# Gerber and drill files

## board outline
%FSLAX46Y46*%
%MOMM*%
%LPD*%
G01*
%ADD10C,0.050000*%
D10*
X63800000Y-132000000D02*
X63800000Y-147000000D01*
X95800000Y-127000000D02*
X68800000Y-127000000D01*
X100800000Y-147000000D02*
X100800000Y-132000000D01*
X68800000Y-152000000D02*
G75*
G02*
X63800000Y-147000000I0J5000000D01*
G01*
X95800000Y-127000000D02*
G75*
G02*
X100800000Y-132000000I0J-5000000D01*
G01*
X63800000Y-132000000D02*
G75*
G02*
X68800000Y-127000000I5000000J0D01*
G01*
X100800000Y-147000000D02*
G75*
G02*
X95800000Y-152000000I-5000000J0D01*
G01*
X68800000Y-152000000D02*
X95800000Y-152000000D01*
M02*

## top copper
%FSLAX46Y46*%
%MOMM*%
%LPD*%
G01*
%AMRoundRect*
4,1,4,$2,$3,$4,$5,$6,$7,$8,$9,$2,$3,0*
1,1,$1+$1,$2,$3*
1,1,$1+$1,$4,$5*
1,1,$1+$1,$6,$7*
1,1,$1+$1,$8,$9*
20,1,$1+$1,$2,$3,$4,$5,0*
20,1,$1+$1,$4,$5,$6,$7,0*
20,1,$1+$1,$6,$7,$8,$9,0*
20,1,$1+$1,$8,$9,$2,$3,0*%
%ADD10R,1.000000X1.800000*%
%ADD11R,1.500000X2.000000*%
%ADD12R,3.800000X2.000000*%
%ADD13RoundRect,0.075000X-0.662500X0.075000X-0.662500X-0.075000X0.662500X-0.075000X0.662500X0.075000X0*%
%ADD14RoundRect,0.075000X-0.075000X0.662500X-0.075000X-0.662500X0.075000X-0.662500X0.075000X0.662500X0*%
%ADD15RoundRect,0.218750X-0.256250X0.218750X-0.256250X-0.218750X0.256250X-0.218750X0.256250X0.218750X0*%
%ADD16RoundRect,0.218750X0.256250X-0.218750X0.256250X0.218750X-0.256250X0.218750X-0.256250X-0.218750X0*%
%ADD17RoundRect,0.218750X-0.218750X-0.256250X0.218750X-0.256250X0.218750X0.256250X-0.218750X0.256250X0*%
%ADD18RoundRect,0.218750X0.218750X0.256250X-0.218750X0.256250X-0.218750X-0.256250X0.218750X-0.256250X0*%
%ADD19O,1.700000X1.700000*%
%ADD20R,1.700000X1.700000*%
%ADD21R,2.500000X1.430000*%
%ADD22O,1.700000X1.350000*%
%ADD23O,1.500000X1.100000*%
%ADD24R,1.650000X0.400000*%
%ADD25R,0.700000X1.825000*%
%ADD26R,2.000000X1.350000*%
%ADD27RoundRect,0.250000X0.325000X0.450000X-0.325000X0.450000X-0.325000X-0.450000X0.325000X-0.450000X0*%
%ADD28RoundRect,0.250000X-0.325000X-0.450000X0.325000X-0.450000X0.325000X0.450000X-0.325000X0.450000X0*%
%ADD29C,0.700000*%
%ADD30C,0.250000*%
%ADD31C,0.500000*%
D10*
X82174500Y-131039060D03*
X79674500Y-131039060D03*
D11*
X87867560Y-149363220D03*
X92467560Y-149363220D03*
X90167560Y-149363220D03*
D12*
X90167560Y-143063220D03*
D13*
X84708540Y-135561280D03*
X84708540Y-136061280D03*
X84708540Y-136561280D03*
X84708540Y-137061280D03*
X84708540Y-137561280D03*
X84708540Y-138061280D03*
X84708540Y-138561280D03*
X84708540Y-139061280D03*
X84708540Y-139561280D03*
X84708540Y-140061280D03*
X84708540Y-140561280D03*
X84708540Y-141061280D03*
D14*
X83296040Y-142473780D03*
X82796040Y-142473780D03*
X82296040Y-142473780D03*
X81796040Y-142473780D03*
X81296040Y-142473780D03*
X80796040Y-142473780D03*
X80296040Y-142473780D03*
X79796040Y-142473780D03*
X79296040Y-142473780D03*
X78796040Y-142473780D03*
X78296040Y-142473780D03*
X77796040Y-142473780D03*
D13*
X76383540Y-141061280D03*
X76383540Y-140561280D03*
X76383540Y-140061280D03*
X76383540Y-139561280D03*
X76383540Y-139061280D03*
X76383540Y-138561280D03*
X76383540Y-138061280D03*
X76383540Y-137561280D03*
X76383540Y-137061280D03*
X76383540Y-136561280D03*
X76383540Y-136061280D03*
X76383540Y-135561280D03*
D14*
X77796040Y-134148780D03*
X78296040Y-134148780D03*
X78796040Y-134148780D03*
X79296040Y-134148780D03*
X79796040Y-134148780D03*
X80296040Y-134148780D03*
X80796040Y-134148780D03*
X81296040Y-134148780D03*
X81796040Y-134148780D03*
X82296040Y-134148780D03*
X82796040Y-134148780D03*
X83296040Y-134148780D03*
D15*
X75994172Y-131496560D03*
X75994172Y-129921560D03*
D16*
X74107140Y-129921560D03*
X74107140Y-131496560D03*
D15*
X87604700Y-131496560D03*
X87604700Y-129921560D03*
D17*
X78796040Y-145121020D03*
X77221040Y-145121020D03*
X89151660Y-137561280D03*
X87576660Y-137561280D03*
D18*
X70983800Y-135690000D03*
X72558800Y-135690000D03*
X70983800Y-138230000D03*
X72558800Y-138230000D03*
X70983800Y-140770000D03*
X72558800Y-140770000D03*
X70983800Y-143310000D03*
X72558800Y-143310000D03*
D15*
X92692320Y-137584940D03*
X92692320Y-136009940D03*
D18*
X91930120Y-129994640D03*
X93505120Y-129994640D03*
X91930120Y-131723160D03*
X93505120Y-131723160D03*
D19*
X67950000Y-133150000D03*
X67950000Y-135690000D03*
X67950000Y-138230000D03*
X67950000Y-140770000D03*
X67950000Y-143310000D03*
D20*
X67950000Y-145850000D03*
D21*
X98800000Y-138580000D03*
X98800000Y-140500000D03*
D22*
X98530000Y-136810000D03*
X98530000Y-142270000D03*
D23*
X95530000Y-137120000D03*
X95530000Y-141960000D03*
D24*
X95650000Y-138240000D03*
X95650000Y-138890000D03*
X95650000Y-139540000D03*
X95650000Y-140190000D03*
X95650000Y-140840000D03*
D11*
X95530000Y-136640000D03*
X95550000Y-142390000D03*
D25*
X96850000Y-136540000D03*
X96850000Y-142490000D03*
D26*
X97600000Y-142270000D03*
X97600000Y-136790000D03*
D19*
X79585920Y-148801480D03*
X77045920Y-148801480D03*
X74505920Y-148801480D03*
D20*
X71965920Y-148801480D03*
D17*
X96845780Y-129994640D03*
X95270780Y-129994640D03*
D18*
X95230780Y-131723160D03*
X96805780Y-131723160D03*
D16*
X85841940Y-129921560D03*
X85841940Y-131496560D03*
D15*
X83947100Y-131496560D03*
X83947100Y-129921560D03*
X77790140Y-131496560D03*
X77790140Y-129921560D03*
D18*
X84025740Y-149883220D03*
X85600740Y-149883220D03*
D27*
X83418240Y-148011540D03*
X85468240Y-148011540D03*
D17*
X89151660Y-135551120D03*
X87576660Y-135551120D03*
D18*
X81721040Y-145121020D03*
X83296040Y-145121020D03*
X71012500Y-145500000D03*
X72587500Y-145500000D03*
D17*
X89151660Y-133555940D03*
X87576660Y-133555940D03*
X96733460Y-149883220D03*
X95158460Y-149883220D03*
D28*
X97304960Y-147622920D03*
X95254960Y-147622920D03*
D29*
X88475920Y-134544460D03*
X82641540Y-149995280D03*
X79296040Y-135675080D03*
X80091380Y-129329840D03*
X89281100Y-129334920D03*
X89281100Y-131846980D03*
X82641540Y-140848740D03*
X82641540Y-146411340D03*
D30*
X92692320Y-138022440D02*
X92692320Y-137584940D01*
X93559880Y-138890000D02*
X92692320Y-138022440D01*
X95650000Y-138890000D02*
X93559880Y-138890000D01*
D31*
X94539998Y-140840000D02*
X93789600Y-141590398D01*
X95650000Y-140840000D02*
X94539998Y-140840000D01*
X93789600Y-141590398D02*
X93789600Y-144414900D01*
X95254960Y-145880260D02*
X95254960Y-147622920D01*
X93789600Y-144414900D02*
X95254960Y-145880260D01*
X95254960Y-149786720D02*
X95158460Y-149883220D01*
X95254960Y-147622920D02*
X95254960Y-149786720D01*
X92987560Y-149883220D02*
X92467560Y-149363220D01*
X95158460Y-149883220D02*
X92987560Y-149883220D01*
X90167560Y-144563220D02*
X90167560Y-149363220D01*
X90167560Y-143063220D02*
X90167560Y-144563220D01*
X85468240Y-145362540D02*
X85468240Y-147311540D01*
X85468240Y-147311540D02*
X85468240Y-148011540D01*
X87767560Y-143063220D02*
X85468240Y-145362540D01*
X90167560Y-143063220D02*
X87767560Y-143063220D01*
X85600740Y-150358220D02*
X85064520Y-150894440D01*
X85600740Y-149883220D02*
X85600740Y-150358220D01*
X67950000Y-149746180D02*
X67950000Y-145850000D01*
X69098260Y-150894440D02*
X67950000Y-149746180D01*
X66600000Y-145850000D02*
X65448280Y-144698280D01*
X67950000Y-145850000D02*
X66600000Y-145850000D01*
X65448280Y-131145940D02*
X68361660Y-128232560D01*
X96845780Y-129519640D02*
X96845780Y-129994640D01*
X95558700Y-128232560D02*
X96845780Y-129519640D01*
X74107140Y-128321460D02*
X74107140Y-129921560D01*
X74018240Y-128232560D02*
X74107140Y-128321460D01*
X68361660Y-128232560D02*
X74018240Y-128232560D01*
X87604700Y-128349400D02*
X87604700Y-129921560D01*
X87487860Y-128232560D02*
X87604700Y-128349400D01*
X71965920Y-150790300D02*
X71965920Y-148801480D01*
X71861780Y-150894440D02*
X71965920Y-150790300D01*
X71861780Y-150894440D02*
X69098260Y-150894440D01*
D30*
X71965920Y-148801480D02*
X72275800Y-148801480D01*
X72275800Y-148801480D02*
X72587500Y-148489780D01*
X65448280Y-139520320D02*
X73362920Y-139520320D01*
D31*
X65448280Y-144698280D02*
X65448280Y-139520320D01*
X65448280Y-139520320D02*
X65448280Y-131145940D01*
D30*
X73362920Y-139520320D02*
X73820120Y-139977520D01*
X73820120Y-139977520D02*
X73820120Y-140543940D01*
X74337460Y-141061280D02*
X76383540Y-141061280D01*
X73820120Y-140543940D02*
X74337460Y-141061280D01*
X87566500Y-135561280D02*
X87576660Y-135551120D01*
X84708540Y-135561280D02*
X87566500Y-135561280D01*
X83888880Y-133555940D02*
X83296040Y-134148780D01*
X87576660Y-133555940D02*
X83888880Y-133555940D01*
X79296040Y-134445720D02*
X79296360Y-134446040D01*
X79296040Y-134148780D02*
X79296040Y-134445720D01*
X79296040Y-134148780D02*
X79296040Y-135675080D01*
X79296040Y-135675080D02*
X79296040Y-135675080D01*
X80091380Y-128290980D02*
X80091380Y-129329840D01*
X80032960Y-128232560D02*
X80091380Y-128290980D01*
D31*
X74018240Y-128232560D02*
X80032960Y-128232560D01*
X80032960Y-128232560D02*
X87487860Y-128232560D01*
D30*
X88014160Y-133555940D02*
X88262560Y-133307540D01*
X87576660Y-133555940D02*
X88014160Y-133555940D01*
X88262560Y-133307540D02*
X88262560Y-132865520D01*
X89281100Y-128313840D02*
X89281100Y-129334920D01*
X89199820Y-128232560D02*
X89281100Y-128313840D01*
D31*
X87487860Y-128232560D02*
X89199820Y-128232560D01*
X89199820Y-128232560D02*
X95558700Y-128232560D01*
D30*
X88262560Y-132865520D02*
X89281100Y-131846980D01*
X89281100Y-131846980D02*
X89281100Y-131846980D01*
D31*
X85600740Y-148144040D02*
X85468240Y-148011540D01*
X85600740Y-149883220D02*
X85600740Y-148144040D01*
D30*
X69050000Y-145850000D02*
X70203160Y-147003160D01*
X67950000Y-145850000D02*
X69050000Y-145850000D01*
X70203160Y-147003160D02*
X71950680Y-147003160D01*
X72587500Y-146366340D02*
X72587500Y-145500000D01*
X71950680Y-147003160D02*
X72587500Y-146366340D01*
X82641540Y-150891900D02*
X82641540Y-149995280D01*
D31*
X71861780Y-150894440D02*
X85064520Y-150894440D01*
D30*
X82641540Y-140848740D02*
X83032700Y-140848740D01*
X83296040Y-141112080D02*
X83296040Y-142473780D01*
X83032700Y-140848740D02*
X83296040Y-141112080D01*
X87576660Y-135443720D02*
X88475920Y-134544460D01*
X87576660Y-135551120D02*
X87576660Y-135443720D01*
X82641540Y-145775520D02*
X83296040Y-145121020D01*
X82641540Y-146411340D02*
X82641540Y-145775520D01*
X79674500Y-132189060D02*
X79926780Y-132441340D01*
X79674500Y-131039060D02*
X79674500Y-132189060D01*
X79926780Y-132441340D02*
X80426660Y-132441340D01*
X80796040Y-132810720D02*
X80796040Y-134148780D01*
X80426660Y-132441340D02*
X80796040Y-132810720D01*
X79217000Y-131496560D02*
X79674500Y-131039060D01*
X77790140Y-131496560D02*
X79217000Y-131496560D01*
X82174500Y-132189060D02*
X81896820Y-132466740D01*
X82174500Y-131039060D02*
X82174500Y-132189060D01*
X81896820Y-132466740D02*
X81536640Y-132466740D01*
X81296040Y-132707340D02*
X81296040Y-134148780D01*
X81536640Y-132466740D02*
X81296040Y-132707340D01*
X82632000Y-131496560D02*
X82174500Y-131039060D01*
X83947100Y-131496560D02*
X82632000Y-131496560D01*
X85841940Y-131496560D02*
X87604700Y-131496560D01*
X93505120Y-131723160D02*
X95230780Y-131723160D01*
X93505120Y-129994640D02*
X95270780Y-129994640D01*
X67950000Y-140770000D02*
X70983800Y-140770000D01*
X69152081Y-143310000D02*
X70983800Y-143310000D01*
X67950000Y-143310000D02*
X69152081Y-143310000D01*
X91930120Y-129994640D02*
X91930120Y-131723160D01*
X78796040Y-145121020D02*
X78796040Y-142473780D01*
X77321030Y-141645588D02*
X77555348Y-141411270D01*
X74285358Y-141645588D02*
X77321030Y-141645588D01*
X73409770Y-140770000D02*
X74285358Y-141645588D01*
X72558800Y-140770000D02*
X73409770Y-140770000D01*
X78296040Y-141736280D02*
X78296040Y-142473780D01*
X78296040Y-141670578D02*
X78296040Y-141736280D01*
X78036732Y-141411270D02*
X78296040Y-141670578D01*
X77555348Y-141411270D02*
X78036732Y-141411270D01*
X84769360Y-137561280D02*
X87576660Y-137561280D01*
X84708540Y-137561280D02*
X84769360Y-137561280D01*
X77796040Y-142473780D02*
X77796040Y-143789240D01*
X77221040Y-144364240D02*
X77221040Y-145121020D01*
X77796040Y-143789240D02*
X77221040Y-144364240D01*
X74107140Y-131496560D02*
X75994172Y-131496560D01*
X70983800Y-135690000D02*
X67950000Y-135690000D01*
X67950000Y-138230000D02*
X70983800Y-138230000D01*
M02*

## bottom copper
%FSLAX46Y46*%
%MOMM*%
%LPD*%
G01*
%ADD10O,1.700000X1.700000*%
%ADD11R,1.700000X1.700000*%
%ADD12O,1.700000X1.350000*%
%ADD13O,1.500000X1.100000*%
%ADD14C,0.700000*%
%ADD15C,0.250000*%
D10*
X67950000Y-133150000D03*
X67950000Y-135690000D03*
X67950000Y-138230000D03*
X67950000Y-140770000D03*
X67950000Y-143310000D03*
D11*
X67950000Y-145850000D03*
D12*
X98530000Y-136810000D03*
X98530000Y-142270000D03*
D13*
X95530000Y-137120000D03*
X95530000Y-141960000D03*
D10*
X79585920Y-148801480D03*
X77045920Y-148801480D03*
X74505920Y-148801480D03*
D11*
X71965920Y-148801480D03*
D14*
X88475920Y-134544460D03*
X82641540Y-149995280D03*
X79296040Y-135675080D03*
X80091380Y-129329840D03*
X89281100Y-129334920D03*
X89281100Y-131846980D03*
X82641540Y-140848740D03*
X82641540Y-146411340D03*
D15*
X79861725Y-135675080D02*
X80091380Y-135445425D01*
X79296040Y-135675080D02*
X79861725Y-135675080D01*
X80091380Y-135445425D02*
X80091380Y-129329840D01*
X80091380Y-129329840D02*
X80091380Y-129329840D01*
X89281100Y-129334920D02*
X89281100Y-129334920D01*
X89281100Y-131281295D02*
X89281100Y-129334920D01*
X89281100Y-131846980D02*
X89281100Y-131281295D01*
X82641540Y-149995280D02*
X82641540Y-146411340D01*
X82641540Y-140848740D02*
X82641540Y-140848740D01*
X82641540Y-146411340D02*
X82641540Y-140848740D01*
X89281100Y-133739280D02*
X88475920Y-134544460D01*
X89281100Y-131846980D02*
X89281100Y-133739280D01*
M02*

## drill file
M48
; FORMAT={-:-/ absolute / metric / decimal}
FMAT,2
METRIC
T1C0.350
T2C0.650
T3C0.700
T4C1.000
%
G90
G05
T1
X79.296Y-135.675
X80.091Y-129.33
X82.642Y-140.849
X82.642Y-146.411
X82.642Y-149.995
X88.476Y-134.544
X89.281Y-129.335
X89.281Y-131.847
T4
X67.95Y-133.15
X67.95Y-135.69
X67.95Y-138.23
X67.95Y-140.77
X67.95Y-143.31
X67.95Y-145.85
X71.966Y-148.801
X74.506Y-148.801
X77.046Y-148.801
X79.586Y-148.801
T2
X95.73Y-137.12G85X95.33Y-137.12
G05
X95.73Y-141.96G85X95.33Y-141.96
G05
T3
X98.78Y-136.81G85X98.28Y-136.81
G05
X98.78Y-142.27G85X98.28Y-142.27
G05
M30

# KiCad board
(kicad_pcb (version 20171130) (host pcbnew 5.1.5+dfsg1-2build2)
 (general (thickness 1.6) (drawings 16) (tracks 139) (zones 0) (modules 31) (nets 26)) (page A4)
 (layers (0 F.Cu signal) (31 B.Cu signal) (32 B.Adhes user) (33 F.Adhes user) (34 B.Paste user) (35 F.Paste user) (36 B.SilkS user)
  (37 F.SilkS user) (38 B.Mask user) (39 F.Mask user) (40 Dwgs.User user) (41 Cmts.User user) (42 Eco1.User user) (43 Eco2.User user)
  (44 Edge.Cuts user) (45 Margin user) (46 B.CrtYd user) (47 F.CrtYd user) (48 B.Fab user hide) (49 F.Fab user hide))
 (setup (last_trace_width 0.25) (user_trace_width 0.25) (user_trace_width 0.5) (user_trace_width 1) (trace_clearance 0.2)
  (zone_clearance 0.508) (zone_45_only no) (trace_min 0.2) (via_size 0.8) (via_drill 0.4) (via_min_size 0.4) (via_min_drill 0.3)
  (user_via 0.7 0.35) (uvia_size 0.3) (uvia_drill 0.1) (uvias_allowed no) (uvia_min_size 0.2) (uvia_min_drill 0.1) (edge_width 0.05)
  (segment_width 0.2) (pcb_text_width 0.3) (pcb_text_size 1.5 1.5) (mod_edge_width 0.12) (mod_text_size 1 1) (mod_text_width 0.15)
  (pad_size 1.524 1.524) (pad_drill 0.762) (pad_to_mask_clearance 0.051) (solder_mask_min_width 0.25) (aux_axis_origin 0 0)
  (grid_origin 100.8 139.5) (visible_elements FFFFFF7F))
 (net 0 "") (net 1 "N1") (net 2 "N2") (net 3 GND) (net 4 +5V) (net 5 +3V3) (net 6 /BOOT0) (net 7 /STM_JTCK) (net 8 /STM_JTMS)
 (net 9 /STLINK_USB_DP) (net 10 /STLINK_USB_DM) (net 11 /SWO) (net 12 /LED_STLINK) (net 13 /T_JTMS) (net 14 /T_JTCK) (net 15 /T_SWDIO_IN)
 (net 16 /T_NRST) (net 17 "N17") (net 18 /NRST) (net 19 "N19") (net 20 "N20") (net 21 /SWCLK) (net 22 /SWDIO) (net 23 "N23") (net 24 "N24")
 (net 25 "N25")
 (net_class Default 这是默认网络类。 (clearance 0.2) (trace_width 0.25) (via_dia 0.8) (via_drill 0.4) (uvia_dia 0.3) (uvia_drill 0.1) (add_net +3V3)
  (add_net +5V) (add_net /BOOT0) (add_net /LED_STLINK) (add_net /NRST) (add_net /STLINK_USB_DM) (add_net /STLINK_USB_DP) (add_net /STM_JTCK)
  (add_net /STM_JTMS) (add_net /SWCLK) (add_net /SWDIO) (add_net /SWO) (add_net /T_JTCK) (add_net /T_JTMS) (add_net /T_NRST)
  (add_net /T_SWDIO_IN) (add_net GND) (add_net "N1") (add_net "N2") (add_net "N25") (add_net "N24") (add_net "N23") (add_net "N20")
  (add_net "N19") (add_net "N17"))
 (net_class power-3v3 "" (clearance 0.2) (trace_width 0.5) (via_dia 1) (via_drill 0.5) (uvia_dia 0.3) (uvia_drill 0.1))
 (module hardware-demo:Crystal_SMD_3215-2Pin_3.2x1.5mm (layer F.Cu) (at 80.9245 131.03906 180)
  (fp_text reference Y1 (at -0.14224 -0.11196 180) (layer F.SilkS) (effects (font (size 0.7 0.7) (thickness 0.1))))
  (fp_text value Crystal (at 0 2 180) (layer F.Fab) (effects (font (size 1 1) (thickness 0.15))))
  (pad 2 smd rect (at -1.25 0 180) (size 1 1.8) (layers F.Cu F.Paste F.Mask) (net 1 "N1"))
  (pad 1 smd rect (at 1.25 0 180) (size 1 1.8) (layers F.Cu F.Paste F.Mask) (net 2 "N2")))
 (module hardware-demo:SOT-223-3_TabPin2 (layer F.Cu) (at 90.16756 146.21322 90)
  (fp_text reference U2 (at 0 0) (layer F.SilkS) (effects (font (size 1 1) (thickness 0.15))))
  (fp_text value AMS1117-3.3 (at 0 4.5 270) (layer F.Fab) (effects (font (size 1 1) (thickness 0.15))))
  (pad 1 smd rect (at -3.15 -2.3 90) (size 2 1.5) (layers F.Cu F.Paste F.Mask) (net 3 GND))
  (pad 3 smd rect (at -3.15 2.3 90) (size 2 1.5) (layers F.Cu F.Paste F.Mask) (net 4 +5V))
  (pad 2 smd rect (at -3.15 0 90) (size 2 1.5) (layers F.Cu F.Paste F.Mask) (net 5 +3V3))
  (pad 2 smd rect (at 3.15 0 90) (size 2 3.8) (layers F.Cu F.Paste F.Mask) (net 5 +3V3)))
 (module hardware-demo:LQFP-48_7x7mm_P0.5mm (layer F.Cu) (at 80.54604 138.31128 270)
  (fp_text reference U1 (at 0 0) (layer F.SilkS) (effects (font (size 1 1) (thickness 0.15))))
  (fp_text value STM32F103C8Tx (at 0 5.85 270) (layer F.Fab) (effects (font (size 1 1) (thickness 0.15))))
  (pad 48 smd roundrect (at -2.75 -4.1625 270) (size 0.3 1.475) (layers F.Cu F.Paste F.Mask) (roundrect_rratio 0.25) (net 5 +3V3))
  (pad 47 smd roundrect (at -2.25 -4.1625 270) (size 0.3 1.475) (layers F.Cu F.Paste F.Mask) (roundrect_rratio 0.25) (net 3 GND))
  (pad 46 smd roundrect (at -1.75 -4.1625 270) (size 0.3 1.475) (layers F.Cu F.Paste F.Mask) (roundrect_rratio 0.25))
  (pad 45 smd roundrect (at -1.25 -4.1625 270) (size 0.3 1.475) (layers F.Cu F.Paste F.Mask) (roundrect_rratio 0.25))
  (pad 44 smd roundrect (at -0.75 -4.1625 270) (size 0.3 1.475) (layers F.Cu F.Paste F.Mask) (roundrect_rratio 0.25) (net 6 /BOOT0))
  (pad 43 smd roundrect (at -0.25 -4.1625 270) (size 0.3 1.475) (layers F.Cu F.Paste F.Mask) (roundrect_rratio 0.25))
  (pad 42 smd roundrect (at 0.25 -4.1625 270) (size 0.3 1.475) (layers F.Cu F.Paste F.Mask) (roundrect_rratio 0.25))
  (pad 41 smd roundrect (at 0.75 -4.1625 270) (size 0.3 1.475) (layers F.Cu F.Paste F.Mask) (roundrect_rratio 0.25))
  (pad 40 smd roundrect (at 1.25 -4.1625 270) (size 0.3 1.475) (layers F.Cu F.Paste F.Mask) (roundrect_rratio 0.25))
  (pad 39 smd roundrect (at 1.75 -4.1625 270) (size 0.3 1.475) (layers F.Cu F.Paste F.Mask) (roundrect_rratio 0.25))
  (pad 38 smd roundrect (at 2.25 -4.1625 270) (size 0.3 1.475) (layers F.Cu F.Paste F.Mask) (roundrect_rratio 0.25))
  (pad 37 smd roundrect (at 2.75 -4.1625 270) (size 0.3 1.475) (layers F.Cu F.Paste F.Mask) (roundrect_rratio 0.25) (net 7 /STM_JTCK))
  (pad 36 smd roundrect (at 4.1625 -2.75 270) (size 1.475 0.3) (layers F.Cu F.Paste F.Mask) (roundrect_rratio 0.25) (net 5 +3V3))
  (pad 35 smd roundrect (at 4.1625 -2.25 270) (size 1.475 0.3) (layers F.Cu F.Paste F.Mask) (roundrect_rratio 0.25) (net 3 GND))
  (pad 34 smd roundrect (at 4.1625 -1.75 270) (size 1.475 0.3) (layers F.Cu F.Paste F.Mask) (roundrect_rratio 0.25) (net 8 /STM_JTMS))
  (pad 33 smd roundrect (at 4.1625 -1.25 270) (size 1.475 0.3) (layers F.Cu F.Paste F.Mask) (roundrect_rratio 0.25) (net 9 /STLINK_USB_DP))
  (pad 32 smd roundrect (at 4.1625 -0.75 270) (size 1.475 0.3) (layers F.Cu F.Paste F.Mask) (roundrect_rratio 0.25) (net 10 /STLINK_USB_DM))
  (pad 31 smd roundrect (at 4.1625 -0.25 270) (size 1.475 0.3) (layers F.Cu F.Paste F.Mask) (roundrect_rratio 0.25) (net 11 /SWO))
  (pad 30 smd roundrect (at 4.1625 0.25 270) (size 1.475 0.3) (layers F.Cu F.Paste F.Mask) (roundrect_rratio 0.25) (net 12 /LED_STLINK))
  (pad 29 smd roundrect (at 4.1625 0.75 270) (size 1.475 0.3) (layers F.Cu F.Paste F.Mask) (roundrect_rratio 0.25))
  (pad 28 smd roundrect (at 4.1625 1.25 270) (size 1.475 0.3) (layers F.Cu F.Paste F.Mask) (roundrect_rratio 0.25))
  (pad 27 smd roundrect (at 4.1625 1.75 270) (size 1.475 0.3) (layers F.Cu F.Paste F.Mask) (roundrect_rratio 0.25) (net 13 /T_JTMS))
  (pad 26 smd roundrect (at 4.1625 2.25 270) (size 1.475 0.3) (layers F.Cu F.Paste F.Mask) (roundrect_rratio 0.25) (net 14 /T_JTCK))
  (pad 25 smd roundrect (at 4.1625 2.75 270) (size 1.475 0.3) (layers F.Cu F.Paste F.Mask) (roundrect_rratio 0.25) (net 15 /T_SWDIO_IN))
  (pad 24 smd roundrect (at 2.75 4.1625 270) (size 0.3 1.475) (layers F.Cu F.Paste F.Mask) (roundrect_rratio 0.25) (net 5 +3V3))
  (pad 23 smd roundrect (at 2.25 4.1625 270) (size 0.3 1.475) (layers F.Cu F.Paste F.Mask) (roundrect_rratio 0.25) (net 3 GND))
  (pad 22 smd roundrect (at 1.75 4.1625 270) (size 0.3 1.475) (layers F.Cu F.Paste F.Mask) (roundrect_rratio 0.25))
  (pad 21 smd roundrect (at 1.25 4.1625 270) (size 0.3 1.475) (layers F.Cu F.Paste F.Mask) (roundrect_rratio 0.25))
  (pad 20 smd roundrect (at 0.75 4.1625 270) (size 0.3 1.475) (layers F.Cu F.Paste F.Mask) (roundrect_rratio 0.25) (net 3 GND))
  (pad 19 smd roundrect (at 0.25 4.1625 270) (size 0.3 1.475) (layers F.Cu F.Paste F.Mask) (roundrect_rratio 0.25))
  (pad 18 smd roundrect (at -0.25 4.1625 270) (size 0.3 1.475) (layers F.Cu F.Paste F.Mask) (roundrect_rratio 0.25) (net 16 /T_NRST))
  (pad 17 smd roundrect (at -0.75 4.1625 270) (size 0.3 1.475) (layers F.Cu F.Paste F.Mask) (roundrect_rratio 0.25))
  (pad 16 smd roundrect (at -1.25 4.1625 270) (size 0.3 1.475) (layers F.Cu F.Paste F.Mask) (roundrect_rratio 0.25))
  (pad 15 smd roundrect (at -1.75 4.1625 270) (size 0.3 1.475) (layers F.Cu F.Paste F.Mask) (roundrect_rratio 0.25) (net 14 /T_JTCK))
  (pad 14 smd roundrect (at -2.25 4.1625 270) (size 0.3 1.475) (layers F.Cu F.Paste F.Mask) (roundrect_rratio 0.25))
  (pad 13 smd roundrect (at -2.75 4.1625 270) (size 0.3 1.475) (layers F.Cu F.Paste F.Mask) (roundrect_rratio 0.25))
  (pad 12 smd roundrect (at -4.1625 2.75 270) (size 1.475 0.3) (layers F.Cu F.Paste F.Mask) (roundrect_rratio 0.25))
  (pad 11 smd roundrect (at -4.1625 2.25 270) (size 1.475 0.3) (layers F.Cu F.Paste F.Mask) (roundrect_rratio 0.25))
  (pad 10 smd roundrect (at -4.1625 1.75 270) (size 1.475 0.3) (layers F.Cu F.Paste F.Mask) (roundrect_rratio 0.25) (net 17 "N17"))
  (pad 9 smd roundrect (at -4.1625 1.25 270) (size 1.475 0.3) (layers F.Cu F.Paste F.Mask) (roundrect_rratio 0.25) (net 5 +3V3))
  (pad 8 smd roundrect (at -4.1625 0.75 270) (size 1.475 0.3) (layers F.Cu F.Paste F.Mask) (roundrect_rratio 0.25) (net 3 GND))
  (pad 7 smd roundrect (at -4.1625 0.25 270) (size 1.475 0.3) (layers F.Cu F.Paste F.Mask) (roundrect_rratio 0.25) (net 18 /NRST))
  (pad 6 smd roundrect (at -4.1625 -0.25 270) (size 1.475 0.3) (layers F.Cu F.Paste F.Mask) (roundrect_rratio 0.25) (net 2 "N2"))
  (pad 5 smd roundrect (at -4.1625 -0.75 270) (size 1.475 0.3) (layers F.Cu F.Paste F.Mask) (roundrect_rratio 0.25) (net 1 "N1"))
  (pad 4 smd roundrect (at -4.1625 -1.25 270) (size 1.475 0.3) (layers F.Cu F.Paste F.Mask) (roundrect_rratio 0.25))
  (pad 3 smd roundrect (at -4.1625 -1.75 270) (size 1.475 0.3) (layers F.Cu F.Paste F.Mask) (roundrect_rratio 0.25))
  (pad 2 smd roundrect (at -4.1625 -2.25 270) (size 1.475 0.3) (layers F.Cu F.Paste F.Mask) (roundrect_rratio 0.25))
  (pad 1 smd roundrect (at -4.1625 -2.75 270) (size 1.475 0.3) (layers F.Cu F.Paste F.Mask) (roundrect_rratio 0.25) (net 5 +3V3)))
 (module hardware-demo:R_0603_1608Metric (layer F.Cu) (at 75.994172 130.70906 270)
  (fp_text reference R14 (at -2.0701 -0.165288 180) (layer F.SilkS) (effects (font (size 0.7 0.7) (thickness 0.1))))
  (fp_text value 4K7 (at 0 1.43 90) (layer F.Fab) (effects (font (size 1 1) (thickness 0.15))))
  (pad 2 smd roundrect (at 0.7875 0 270) (size 0.875 0.95) (layers F.Cu F.Paste F.Mask) (roundrect_rratio 0.25) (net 17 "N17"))
  (pad 1 smd roundrect (at -0.7875 0 270) (size 0.875 0.95) (layers F.Cu F.Paste F.Mask) (roundrect_rratio 0.25) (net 3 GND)))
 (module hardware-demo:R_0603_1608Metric (layer F.Cu) (at 74.10714 130.70906 90)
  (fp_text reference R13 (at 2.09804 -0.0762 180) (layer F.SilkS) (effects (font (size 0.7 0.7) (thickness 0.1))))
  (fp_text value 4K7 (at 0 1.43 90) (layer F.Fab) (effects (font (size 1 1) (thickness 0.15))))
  (pad 2 smd roundrect (at 0.7875 0 90) (size 0.875 0.95) (layers F.Cu F.Paste F.Mask) (roundrect_rratio 0.25) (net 5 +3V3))
  (pad 1 smd roundrect (at -0.7875 0 90) (size 0.875 0.95) (layers F.Cu F.Paste F.Mask) (roundrect_rratio 0.25) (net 17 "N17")))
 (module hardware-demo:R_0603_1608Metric (layer F.Cu) (at 87.6047 130.70906 270)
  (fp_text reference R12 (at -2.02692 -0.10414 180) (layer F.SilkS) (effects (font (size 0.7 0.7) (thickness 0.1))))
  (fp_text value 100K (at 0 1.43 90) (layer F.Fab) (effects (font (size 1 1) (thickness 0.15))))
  (pad 2 smd roundrect (at 0.7875 0 270) (size 0.875 0.95) (layers F.Cu F.Paste F.Mask) (roundrect_rratio 0.25) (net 18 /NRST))
  (pad 1 smd roundrect (at -0.7875 0 270) (size 0.875 0.95) (layers F.Cu F.Paste F.Mask) (roundrect_rratio 0.25) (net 5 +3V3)))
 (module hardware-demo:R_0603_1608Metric (layer F.Cu) (at 78.00854 145.12102)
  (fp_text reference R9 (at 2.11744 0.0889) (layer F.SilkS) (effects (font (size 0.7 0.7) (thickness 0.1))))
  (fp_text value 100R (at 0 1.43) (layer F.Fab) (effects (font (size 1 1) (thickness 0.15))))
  (pad 2 smd roundrect (at 0.7875 0) (size 0.875 0.95) (layers F.Cu F.Paste F.Mask) (roundrect_rratio 0.25) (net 13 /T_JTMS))
  (pad 1 smd roundrect (at -0.7875 0) (size 0.875 0.95) (layers F.Cu F.Paste F.Mask) (roundrect_rratio 0.25) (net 15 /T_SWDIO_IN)))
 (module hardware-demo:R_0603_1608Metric (layer F.Cu) (at 88.36416 137.56128)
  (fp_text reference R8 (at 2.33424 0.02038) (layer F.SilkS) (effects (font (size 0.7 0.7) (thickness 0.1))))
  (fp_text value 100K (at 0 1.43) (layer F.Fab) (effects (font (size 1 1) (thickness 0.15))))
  (pad 2 smd roundrect (at 0.7875 0) (size 0.875 0.95) (layers F.Cu F.Paste F.Mask) (roundrect_rratio 0.25) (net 3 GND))
  (pad 1 smd roundrect (at -0.7875 0) (size 0.875 0.95) (layers F.Cu F.Paste F.Mask) (roundrect_rratio 0.25) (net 6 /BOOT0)))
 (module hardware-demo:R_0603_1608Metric (layer F.Cu) (at 71.7713 135.69 180)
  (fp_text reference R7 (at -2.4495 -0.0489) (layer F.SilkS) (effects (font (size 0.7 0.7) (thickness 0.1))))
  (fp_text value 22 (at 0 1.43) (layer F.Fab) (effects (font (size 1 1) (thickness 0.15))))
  (pad 2 smd roundrect (at 0.7875 0 180) (size 0.875 0.95) (layers F.Cu F.Paste F.Mask) (roundrect_rratio 0.25) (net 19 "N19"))
  (pad 1 smd roundrect (at -0.7875 0 180) (size 0.875 0.95) (layers F.Cu F.Paste F.Mask) (roundrect_rratio 0.25) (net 11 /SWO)))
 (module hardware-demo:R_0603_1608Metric (layer F.Cu) (at 71.7713 138.23 180)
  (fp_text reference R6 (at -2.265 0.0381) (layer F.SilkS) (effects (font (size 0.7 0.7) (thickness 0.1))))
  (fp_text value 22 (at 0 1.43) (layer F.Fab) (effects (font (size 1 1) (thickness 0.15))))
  (pad 2 smd roundrect (at 0.7875 0 180) (size 0.875 0.95) (layers F.Cu F.Paste F.Mask) (roundrect_rratio 0.25) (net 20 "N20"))
  (pad 1 smd roundrect (at -0.7875 0 180) (size 0.875 0.95) (layers F.Cu F.Paste F.Mask) (roundrect_rratio 0.25) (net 16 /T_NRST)))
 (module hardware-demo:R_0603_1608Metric (layer F.Cu) (at 71.7713 140.77 180)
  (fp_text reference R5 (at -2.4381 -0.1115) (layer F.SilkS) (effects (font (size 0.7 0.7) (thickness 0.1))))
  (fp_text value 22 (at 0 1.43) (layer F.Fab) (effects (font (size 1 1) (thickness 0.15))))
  (pad 2 smd roundrect (at 0.7875 0 180) (size 0.875 0.95) (layers F.Cu F.Paste F.Mask) (roundrect_rratio 0.25) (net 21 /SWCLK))
  (pad 1 smd roundrect (at -0.7875 0 180) (size 0.875 0.95) (layers F.Cu F.Paste F.Mask) (roundrect_rratio 0.25) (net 14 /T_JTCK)))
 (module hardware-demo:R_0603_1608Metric (layer F.Cu) (at 71.7713 143.31 180)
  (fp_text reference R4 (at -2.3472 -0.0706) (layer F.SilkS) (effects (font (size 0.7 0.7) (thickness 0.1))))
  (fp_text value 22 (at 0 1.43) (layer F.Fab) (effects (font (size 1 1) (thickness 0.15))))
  (pad 2 smd roundrect (at 0.7875 0 180) (size 0.875 0.95) (layers F.Cu F.Paste F.Mask) (roundrect_rratio 0.25) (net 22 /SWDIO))
  (pad 1 smd roundrect (at -0.7875 0 180) (size 0.875 0.95) (layers F.Cu F.Paste F.Mask) (roundrect_rratio 0.25) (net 13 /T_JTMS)))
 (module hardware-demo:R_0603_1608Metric (layer F.Cu) (at 92.69232 136.79744 270)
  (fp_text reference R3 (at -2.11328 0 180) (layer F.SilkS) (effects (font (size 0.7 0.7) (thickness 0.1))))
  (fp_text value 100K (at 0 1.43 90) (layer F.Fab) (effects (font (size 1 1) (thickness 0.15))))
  (pad 2 smd roundrect (at 0.7875 0 270) (size 0.875 0.95) (layers F.Cu F.Paste F.Mask) (roundrect_rratio 0.25) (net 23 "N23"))
  (pad 1 smd roundrect (at -0.7875 0 270) (size 0.875 0.95) (layers F.Cu F.Paste F.Mask) (roundrect_rratio 0.25) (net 3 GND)))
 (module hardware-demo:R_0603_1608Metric (layer F.Cu) (at 92.71762 129.99464 180)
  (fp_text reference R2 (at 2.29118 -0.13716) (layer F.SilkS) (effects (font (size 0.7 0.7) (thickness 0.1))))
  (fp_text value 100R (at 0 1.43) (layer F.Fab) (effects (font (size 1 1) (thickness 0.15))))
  (pad 2 smd roundrect (at 0.7875 0 180) (size 0.875 0.95) (layers F.Cu F.Paste F.Mask) (roundrect_rratio 0.25) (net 12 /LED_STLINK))
  (pad 1 smd roundrect (at -0.7875 0 180) (size 0.875 0.95) (layers F.Cu F.Paste F.Mask) (roundrect_rratio 0.25) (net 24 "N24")))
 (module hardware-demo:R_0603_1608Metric (layer F.Cu) (at 92.71762 131.72316 180)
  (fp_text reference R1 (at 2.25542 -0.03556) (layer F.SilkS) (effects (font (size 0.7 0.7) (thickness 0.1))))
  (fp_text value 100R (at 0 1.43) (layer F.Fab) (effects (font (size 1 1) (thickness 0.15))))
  (pad 2 smd roundrect (at 0.7875 0 180) (size 0.875 0.95) (layers F.Cu F.Paste F.Mask) (roundrect_rratio 0.25) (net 12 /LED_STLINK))
  (pad 1 smd roundrect (at -0.7875 0 180) (size 0.875 0.95) (layers F.Cu F.Paste F.Mask) (roundrect_rratio 0.25) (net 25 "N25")))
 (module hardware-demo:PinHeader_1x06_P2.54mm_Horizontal (layer F.Cu) (at 67.95 145.85 180)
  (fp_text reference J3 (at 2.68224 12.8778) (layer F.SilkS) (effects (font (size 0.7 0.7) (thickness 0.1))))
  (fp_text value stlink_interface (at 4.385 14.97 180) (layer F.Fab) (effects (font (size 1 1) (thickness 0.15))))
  (pad 6 thru_hole oval (at 0 12.7 180) (size 1.7 1.7) (drill 1) (layers *.Cu *.Mask) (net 3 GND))
  (pad 5 thru_hole oval (at 0 10.16 180) (size 1.7 1.7) (drill 1) (layers *.Cu *.Mask) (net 19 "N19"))
  (pad 4 thru_hole oval (at 0 7.62 180) (size 1.7 1.7) (drill 1) (layers *.Cu *.Mask) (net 20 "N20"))
  (pad 3 thru_hole oval (at 0 5.08 180) (size 1.7 1.7) (drill 1) (layers *.Cu *.Mask) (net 21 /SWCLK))
  (pad 2 thru_hole oval (at 0 2.54 180) (size 1.7 1.7) (drill 1) (layers *.Cu *.Mask) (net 22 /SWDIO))
  (pad 1 thru_hole rect (at 0 0 180) (size 1.7 1.7) (drill 1) (layers *.Cu *.Mask) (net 5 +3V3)))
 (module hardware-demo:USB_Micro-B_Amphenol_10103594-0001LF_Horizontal (layer F.Cu) (at 97.415 139.515 90)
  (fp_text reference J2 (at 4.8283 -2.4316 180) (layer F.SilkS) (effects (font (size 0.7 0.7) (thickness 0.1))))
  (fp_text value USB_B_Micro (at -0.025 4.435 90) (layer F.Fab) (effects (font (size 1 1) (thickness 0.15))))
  (pad 6 smd rect (at 0.935 1.385 180) (size 2.5 1.43) (layers F.Cu F.Paste F.Mask) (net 3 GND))
  (pad 6 smd rect (at -0.985 1.385 180) (size 2.5 1.43) (layers F.Cu F.Paste F.Mask) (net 3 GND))
  (pad 6 thru_hole oval (at 2.705 1.115 180) (size 1.7 1.35) (drill oval 1.2 0.7) (layers *.Cu *.Mask) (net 3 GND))
  (pad 6 thru_hole oval (at -2.755 1.115 180) (size 1.7 1.35) (drill oval 1.2 0.7) (layers *.Cu *.Mask) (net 3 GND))
  (pad 6 thru_hole oval (at 2.395 -1.885 180) (size 1.5 1.1) (drill oval 1.05 0.65) (layers *.Cu *.Mask) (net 3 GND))
  (pad 6 thru_hole oval (at -2.445 -1.885 180) (size 1.5 1.1) (drill oval 1.05 0.65) (layers *.Cu *.Mask) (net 3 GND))
  (pad 5 smd rect (at 1.275 -1.765 180) (size 1.65 0.4) (layers F.Cu F.Paste F.Mask) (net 3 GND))
  (pad 4 smd rect (at 0.625 -1.765 180) (size 1.65 0.4) (layers F.Cu F.Paste F.Mask) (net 23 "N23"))
  (pad 3 smd rect (at -0.025 -1.765 180) (size 1.65 0.4) (layers F.Cu F.Paste F.Mask) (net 9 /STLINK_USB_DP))
  (pad 2 smd rect (at -0.675 -1.765 180) (size 1.65 0.4) (layers F.Cu F.Paste F.Mask) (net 10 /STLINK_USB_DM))
  (pad 1 smd rect (at -1.325 -1.765 180) (size 1.65 0.4) (layers F.Cu F.Paste F.Mask) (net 4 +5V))
  (pad 6 smd rect (at 2.875 -1.885 90) (size 2 1.5) (layers F.Cu F.Paste F.Mask) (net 3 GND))
  (pad 6 smd rect (at -2.875 -1.865 90) (size 2 1.5) (layers F.Cu F.Paste F.Mask) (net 3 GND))
  (pad 6 smd rect (at 2.975 -0.565 90) (size 1.825 0.7) (layers F.Cu F.Paste F.Mask) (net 3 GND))
  (pad 6 smd rect (at -2.975 -0.565 90) (size 1.825 0.7) (layers F.Cu F.Paste F.Mask) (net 3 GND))
  (pad 6 smd rect (at -2.755 0.185 90) (size 1.35 2) (layers F.Cu F.Paste F.Mask) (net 3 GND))
  (pad 6 smd rect (at 2.725 0.185 90) (size 1.35 2) (layers F.Cu F.Paste F.Mask) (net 3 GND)))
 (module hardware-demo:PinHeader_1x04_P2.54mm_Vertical (layer F.Cu) (at 71.96592 148.80148 90)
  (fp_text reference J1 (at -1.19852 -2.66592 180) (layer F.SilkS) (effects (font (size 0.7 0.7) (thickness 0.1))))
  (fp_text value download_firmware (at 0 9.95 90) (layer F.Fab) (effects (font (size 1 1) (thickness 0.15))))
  (pad 4 thru_hole oval (at 0 7.62 90) (size 1.7 1.7) (drill 1) (layers *.Cu *.Mask) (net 3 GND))
  (pad 3 thru_hole oval (at 0 5.08 90) (size 1.7 1.7) (drill 1) (layers *.Cu *.Mask) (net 7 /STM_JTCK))
  (pad 2 thru_hole oval (at 0 2.54 90) (size 1.7 1.7) (drill 1) (layers *.Cu *.Mask) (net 8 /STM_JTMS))
  (pad 1 thru_hole rect (at 0 0 90) (size 1.7 1.7) (drill 1) (layers *.Cu *.Mask) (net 5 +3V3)))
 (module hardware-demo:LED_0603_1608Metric (layer F.Cu) (at 96.05828 129.99464)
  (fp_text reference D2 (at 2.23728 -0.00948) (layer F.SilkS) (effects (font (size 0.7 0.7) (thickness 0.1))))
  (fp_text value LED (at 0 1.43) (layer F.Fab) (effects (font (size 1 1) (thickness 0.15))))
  (pad 2 smd roundrect (at 0.7875 0) (size 0.875 0.95) (layers F.Cu F.Paste F.Mask) (roundrect_rratio 0.25) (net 5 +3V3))
  (pad 1 smd roundrect (at -0.7875 0) (size 0.875 0.95) (layers F.Cu F.Paste F.Mask) (roundrect_rratio 0.25) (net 24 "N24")))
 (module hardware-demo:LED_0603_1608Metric (layer F.Cu) (at 96.01828 131.72316 180)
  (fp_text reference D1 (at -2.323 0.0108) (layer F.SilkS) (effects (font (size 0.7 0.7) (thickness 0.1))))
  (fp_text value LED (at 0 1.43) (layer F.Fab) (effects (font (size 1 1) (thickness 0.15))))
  (pad 2 smd roundrect (at 0.7875 0 180) (size 0.875 0.95) (layers F.Cu F.Paste F.Mask) (roundrect_rratio 0.25) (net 25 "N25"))
  (pad 1 smd roundrect (at -0.7875 0 180) (size 0.875 0.95) (layers F.Cu F.Paste F.Mask) (roundrect_rratio 0.25) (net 3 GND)))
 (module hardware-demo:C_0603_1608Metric (layer F.Cu) (at 85.84194 130.70906 90)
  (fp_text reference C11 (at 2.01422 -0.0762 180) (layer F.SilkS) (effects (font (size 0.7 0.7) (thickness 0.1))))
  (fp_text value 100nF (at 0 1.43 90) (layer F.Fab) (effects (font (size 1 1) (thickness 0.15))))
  (pad 2 smd roundrect (at 0.7875 0 90) (size 0.875 0.95) (layers F.Cu F.Paste F.Mask) (roundrect_rratio 0.25) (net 3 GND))
  (pad 1 smd roundrect (at -0.7875 0 90) (size 0.875 0.95) (layers F.Cu F.Paste F.Mask) (roundrect_rratio 0.25) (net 18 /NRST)))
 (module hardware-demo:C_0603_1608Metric (layer F.Cu) (at 83.9471 130.70906 270)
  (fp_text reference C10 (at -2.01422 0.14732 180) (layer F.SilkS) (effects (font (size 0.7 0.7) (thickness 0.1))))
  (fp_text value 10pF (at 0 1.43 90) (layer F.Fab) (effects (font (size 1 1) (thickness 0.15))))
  (pad 2 smd roundrect (at 0.7875 0 270) (size 0.875 0.95) (layers F.Cu F.Paste F.Mask) (roundrect_rratio 0.25) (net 1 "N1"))
  (pad 1 smd roundrect (at -0.7875 0 270) (size 0.875 0.95) (layers F.Cu F.Paste F.Mask) (roundrect_rratio 0.25) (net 3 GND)))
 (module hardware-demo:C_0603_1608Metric (layer F.Cu) (at 77.79014 130.70906 270)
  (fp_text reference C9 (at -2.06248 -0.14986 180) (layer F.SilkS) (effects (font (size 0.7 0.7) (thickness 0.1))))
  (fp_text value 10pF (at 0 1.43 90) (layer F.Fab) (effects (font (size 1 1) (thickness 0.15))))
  (pad 2 smd roundrect (at 0.7875 0 270) (size 0.875 0.95) (layers F.Cu F.Paste F.Mask) (roundrect_rratio 0.25) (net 2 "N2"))
  (pad 1 smd roundrect (at -0.7875 0 270) (size 0.875 0.95) (layers F.Cu F.Paste F.Mask) (roundrect_rratio 0.25) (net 3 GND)))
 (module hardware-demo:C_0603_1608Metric (layer F.Cu) (at 84.81324 149.88322 180)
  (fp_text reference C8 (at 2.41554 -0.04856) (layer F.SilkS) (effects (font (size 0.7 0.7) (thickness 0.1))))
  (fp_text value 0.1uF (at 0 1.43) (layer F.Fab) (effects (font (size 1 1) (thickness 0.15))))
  (pad 2 smd roundrect (at 0.7875 0 180) (size 0.875 0.95) (layers F.Cu F.Paste F.Mask) (roundrect_rratio 0.25) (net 3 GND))
  (pad 1 smd roundrect (at -0.7875 0 180) (size 0.875 0.95) (layers F.Cu F.Paste F.Mask) (roundrect_rratio 0.25) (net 5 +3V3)))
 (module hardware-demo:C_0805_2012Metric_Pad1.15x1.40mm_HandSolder (layer F.Cu) (at 84.44324 148.01154 180)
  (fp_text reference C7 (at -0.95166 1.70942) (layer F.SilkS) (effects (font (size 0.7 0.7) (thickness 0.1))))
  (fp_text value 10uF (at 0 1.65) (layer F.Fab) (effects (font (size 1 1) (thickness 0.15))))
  (pad 2 smd roundrect (at 1.025 0 180) (size 1.15 1.4) (layers F.Cu F.Paste F.Mask) (roundrect_rratio 0.217391) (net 3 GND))
  (pad 1 smd roundrect (at -1.025 0 180) (size 1.15 1.4) (layers F.Cu F.Paste F.Mask) (roundrect_rratio 0.217391) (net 5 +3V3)))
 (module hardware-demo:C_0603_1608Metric (layer F.Cu) (at 88.36416 135.55112)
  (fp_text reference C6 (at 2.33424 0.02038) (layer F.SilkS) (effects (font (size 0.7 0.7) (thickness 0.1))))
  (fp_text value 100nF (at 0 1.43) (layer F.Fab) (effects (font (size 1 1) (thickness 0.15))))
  (pad 2 smd roundrect (at 0.7875 0) (size 0.875 0.95) (layers F.Cu F.Paste F.Mask) (roundrect_rratio 0.25) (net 3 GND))
  (pad 1 smd roundrect (at -0.7875 0) (size 0.875 0.95) (layers F.Cu F.Paste F.Mask) (roundrect_rratio 0.25) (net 5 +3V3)))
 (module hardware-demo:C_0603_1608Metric (layer F.Cu) (at 82.50854 145.12102 180)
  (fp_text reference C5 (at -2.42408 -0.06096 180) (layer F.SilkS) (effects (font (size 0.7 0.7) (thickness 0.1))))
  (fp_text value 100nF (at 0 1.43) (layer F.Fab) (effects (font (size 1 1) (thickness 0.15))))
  (pad 2 smd roundrect (at 0.7875 0 180) (size 0.875 0.95) (layers F.Cu F.Paste F.Mask) (roundrect_rratio 0.25) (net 3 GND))
  (pad 1 smd roundrect (at -0.7875 0 180) (size 0.875 0.95) (layers F.Cu F.Paste F.Mask) (roundrect_rratio 0.25) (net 5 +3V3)))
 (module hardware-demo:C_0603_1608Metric (layer F.Cu) (at 71.8 145.5 180)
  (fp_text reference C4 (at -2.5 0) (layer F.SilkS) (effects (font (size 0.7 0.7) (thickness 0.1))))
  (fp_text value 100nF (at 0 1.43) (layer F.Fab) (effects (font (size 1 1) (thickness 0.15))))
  (pad 2 smd roundrect (at 0.7875 0 180) (size 0.875 0.95) (layers F.Cu F.Paste F.Mask) (roundrect_rratio 0.25) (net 3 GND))
  (pad 1 smd roundrect (at -0.7875 0 180) (size 0.875 0.95) (layers F.Cu F.Paste F.Mask) (roundrect_rratio 0.25) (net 5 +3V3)))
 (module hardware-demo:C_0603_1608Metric (layer F.Cu) (at 88.36416 133.55594)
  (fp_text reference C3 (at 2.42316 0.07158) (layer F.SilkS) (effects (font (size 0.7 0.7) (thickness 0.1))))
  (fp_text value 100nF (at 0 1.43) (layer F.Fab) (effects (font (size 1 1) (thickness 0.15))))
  (pad 2 smd roundrect (at 0.7875 0) (size 0.875 0.95) (layers F.Cu F.Paste F.Mask) (roundrect_rratio 0.25) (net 3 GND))
  (pad 1 smd roundrect (at -0.7875 0) (size 0.875 0.95) (layers F.Cu F.Paste F.Mask) (roundrect_rratio 0.25) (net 5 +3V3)))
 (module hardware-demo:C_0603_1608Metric (layer F.Cu) (at 95.94596 149.88322)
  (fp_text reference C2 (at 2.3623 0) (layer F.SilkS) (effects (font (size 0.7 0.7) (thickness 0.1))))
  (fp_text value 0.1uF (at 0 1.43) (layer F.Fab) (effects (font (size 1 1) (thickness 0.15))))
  (pad 2 smd roundrect (at 0.7875 0) (size 0.875 0.95) (layers F.Cu F.Paste F.Mask) (roundrect_rratio 0.25) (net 3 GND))
  (pad 1 smd roundrect (at -0.7875 0) (size 0.875 0.95) (layers F.Cu F.Paste F.Mask) (roundrect_rratio 0.25) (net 4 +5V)))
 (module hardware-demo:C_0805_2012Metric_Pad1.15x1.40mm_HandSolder (layer F.Cu) (at 96.27996 147.62292)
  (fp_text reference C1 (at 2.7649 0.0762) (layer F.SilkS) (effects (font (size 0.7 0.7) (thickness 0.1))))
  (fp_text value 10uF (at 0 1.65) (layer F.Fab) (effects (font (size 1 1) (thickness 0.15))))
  (pad 2 smd roundrect (at 1.025 0) (size 1.15 1.4) (layers F.Cu F.Paste F.Mask) (roundrect_rratio 0.217391) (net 3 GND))
  (pad 1 smd roundrect (at -1.025 0) (size 1.15 1.4) (layers F.Cu F.Paste F.Mask) (roundrect_rratio 0.217391) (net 4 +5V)))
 (gr_line (start 63.8 132) (end 63.8 147) (layer Edge.Cuts) (width 0.05))
 (gr_line (start 95.8 127) (end 68.8 127) (layer Edge.Cuts) (width 0.05))
 (gr_line (start 100.8 147) (end 100.8 132) (layer Edge.Cuts) (width 0.05))
 (gr_arc (start 68.8 147) (end 63.8 147) (angle -90) (layer Edge.Cuts) (width 0.05))
 (gr_arc (start 95.8 132) (end 100.8 132) (angle -90) (layer Edge.Cuts) (width 0.05))
 (gr_arc (start 68.8 132) (end 68.8 127) (angle -90) (layer Edge.Cuts) (width 0.05))
 (gr_arc (start 95.8 147) (end 95.8 152) (angle -90) (layer Edge.Cuts) (width 0.05))
 (gr_line (start 68.8 152) (end 95.8 152) (layer Edge.Cuts) (width 0.05))
 (via (at 88.47592 134.54446) (size 0.7) (drill 0.35) (layers F.Cu B.Cu) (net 5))
 (via micro (at 82.64154 149.99528) (size 0.7) (drill 0.35) (layers F.Cu B.Cu) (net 5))
 (segment (start 92.69232 138.02244) (end 92.69232 137.58494) (width 0.25) (layer F.Cu) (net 23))
 (segment (start 93.55988 138.89) (end 92.69232 138.02244) (width 0.25) (layer F.Cu) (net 23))
 (segment (start 95.65 138.89) (end 93.55988 138.89) (width 0.25) (layer F.Cu) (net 23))
 (segment (start 94.539998 140.84) (end 93.7896 141.590398) (width 0.5) (layer F.Cu) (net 4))
 (segment (start 95.65 140.84) (end 94.539998 140.84) (width 0.5) (layer F.Cu) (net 4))
 (segment (start 93.7896 141.590398) (end 93.7896 144.4149) (width 0.5) (layer F.Cu) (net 4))
 (segment (start 95.25496 145.88026) (end 95.25496 147.62292) (width 0.5) (layer F.Cu) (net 4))
 (segment (start 93.7896 144.4149) (end 95.25496 145.88026) (width 0.5) (layer F.Cu) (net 4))
 (segment (start 95.25496 149.78672) (end 95.15846 149.88322) (width 0.5) (layer F.Cu) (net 4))
 (segment (start 95.25496 147.62292) (end 95.25496 149.78672) (width 0.5) (layer F.Cu) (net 4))
 (segment (start 92.98756 149.88322) (end 92.46756 149.36322) (width 0.5) (layer F.Cu) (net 4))
 (segment (start 95.15846 149.88322) (end 92.98756 149.88322) (width 0.5) (layer F.Cu) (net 4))
 (segment (start 90.16756 144.56322) (end 90.16756 149.36322) (width 0.5) (layer F.Cu) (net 5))
 (segment (start 90.16756 143.06322) (end 90.16756 144.56322) (width 0.5) (layer F.Cu) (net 5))
 (segment (start 85.46824 145.36254) (end 85.46824 147.31154) (width 0.5) (layer F.Cu) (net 5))
 (segment (start 85.46824 147.31154) (end 85.46824 148.01154) (width 0.5) (layer F.Cu) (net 5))
 (segment (start 87.76756 143.06322) (end 85.46824 145.36254) (width 0.5) (layer F.Cu) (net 5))
 (segment (start 90.16756 143.06322) (end 87.76756 143.06322) (width 0.5) (layer F.Cu) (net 5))
 (segment (start 85.60074 150.35822) (end 85.06452 150.89444) (width 0.5) (layer F.Cu) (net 5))
 (segment (start 85.60074 149.88322) (end 85.60074 150.35822) (width 0.5) (layer F.Cu) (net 5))
 (segment (start 67.95 149.74618) (end 67.95 145.85) (width 0.5) (layer F.Cu) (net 5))
 (segment (start 69.09826 150.89444) (end 67.95 149.74618) (width 0.5) (layer F.Cu) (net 5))
 (segment (start 66.6 145.85) (end 65.44828 144.69828) (width 0.5) (layer F.Cu) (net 5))
 (segment (start 67.95 145.85) (end 66.6 145.85) (width 0.5) (layer F.Cu) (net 5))
 (segment (start 65.44828 131.14594) (end 68.36166 128.23256) (width 0.5) (layer F.Cu) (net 5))
 (segment (start 96.84578 129.51964) (end 96.84578 129.99464) (width 0.5) (layer F.Cu) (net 5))
 (segment (start 95.5587 128.23256) (end 96.84578 129.51964) (width 0.5) (layer F.Cu) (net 5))
 (segment (start 74.10714 128.32146) (end 74.10714 129.92156) (width 0.5) (layer F.Cu) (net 5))
 (segment (start 74.01824 128.23256) (end 74.10714 128.32146) (width 0.5) (layer F.Cu) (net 5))
 (segment (start 68.36166 128.23256) (end 74.01824 128.23256) (width 0.5) (layer F.Cu) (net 5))
 (segment (start 87.6047 128.3494) (end 87.6047 129.92156) (width 0.5) (layer F.Cu) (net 5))
 (segment (start 87.48786 128.23256) (end 87.6047 128.3494) (width 0.5) (layer F.Cu) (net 5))
 (segment (start 71.96592 150.7903) (end 71.96592 148.80148) (width 0.5) (layer F.Cu) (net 5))
 (segment (start 71.86178 150.89444) (end 71.96592 150.7903) (width 0.5) (layer F.Cu) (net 5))
 (segment (start 71.86178 150.89444) (end 69.09826 150.89444) (width 0.5) (layer F.Cu) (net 5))
 (segment (start 71.96592 148.80148) (end 72.2758 148.80148) (width 0.25) (layer F.Cu) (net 5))
 (segment (start 72.2758 148.80148) (end 72.5875 148.48978) (width 0.25) (layer F.Cu) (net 5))
 (segment (start 65.44828 139.52032) (end 73.36292 139.52032) (width 0.25) (layer F.Cu) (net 5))
 (segment (start 65.44828 144.69828) (end 65.44828 139.52032) (width 0.5) (layer F.Cu) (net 5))
 (segment (start 65.44828 139.52032) (end 65.44828 131.14594) (width 0.5) (layer F.Cu) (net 5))
 (segment (start 73.36292 139.52032) (end 73.82012 139.97752) (width 0.25) (layer F.Cu) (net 5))
 (segment (start 73.82012 139.97752) (end 73.82012 140.54394) (width 0.25) (layer F.Cu) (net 5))
 (segment (start 74.33746 141.06128) (end 76.38354 141.06128) (width 0.25) (layer F.Cu) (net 5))
 (segment (start 73.82012 140.54394) (end 74.33746 141.06128) (width 0.25) (layer F.Cu) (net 5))
 (segment (start 87.5665 135.56128) (end 87.57666 135.55112) (width 0.25) (layer F.Cu) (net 5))
 (segment (start 84.70854 135.56128) (end 87.5665 135.56128) (width 0.25) (layer F.Cu) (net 5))
 (segment (start 83.88888 133.55594) (end 83.29604 134.14878) (width 0.25) (layer F.Cu) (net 5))
 (segment (start 87.57666 133.55594) (end 83.88888 133.55594) (width 0.25) (layer F.Cu) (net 5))
 (segment (start 79.29604 134.44572) (end 79.29636 134.44604) (width 0.25) (layer F.Cu) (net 5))
 (segment (start 79.29604 134.14878) (end 79.29604 134.44572) (width 0.25) (layer F.Cu) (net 5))
 (segment (start 79.29604 134.14878) (end 79.29604 135.67508) (width 0.25) (layer F.Cu) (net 5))
 (segment (start 79.29604 135.67508) (end 79.29604 135.67508) (width 0.25) (layer F.Cu) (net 5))
 (via micro (at 79.29604 135.67508) (size 0.7) (drill 0.35) (layers F.Cu B.Cu) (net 5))
 (segment (start 79.861725 135.67508) (end 80.09138 135.445425) (width 0.25) (layer B.Cu) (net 5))
 (segment (start 79.29604 135.67508) (end 79.861725 135.67508) (width 0.25) (layer B.Cu) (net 5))
 (segment (start 80.09138 135.445425) (end 80.09138 129.32984) (width 0.25) (layer B.Cu) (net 5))
 (segment (start 80.09138 129.32984) (end 80.09138 129.32984) (width 0.25) (layer B.Cu) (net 5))
 (via micro (at 80.09138 129.32984) (size 0.7) (drill 0.35) (layers F.Cu B.Cu) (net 5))
 (segment (start 80.09138 128.29098) (end 80.09138 129.32984) (width 0.25) (layer F.Cu) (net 5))
 (segment (start 80.03296 128.23256) (end 80.09138 128.29098) (width 0.25) (layer F.Cu) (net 5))
 (segment (start 74.01824 128.23256) (end 80.03296 128.23256) (width 0.5) (layer F.Cu) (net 5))
 (segment (start 80.03296 128.23256) (end 87.48786 128.23256) (width 0.5) (layer F.Cu) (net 5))
 (segment (start 88.01416 133.55594) (end 88.26256 133.30754) (width 0.25) (layer F.Cu) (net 5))
 (segment (start 87.57666 133.55594) (end 88.01416 133.55594) (width 0.25) (layer F.Cu) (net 5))
 (segment (start 88.26256 133.30754) (end 88.26256 132.86552) (width 0.25) (layer F.Cu) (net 5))
 (segment (start 89.2811 129.33492) (end 89.2811 129.33492) (width 0.25) (layer B.Cu) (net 5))
 (via micro (at 89.2811 129.33492) (size 0.7) (drill 0.35) (layers F.Cu B.Cu) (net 5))
 (segment (start 89.2811 128.31384) (end 89.2811 129.33492) (width 0.25) (layer F.Cu) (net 5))
 (segment (start 89.19982 128.23256) (end 89.2811 128.31384) (width 0.25) (layer F.Cu) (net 5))
 (segment (start 87.48786 128.23256) (end 89.19982 128.23256) (width 0.5) (layer F.Cu) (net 5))
 (segment (start 89.19982 128.23256) (end 95.5587 128.23256) (width 0.5) (layer F.Cu) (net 5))
 (segment (start 88.26256 132.86552) (end 89.2811 131.84698) (width 0.25) (layer F.Cu) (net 5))
 (segment (start 89.2811 131.84698) (end 89.2811 131.84698) (width 0.25) (layer F.Cu) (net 5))
 (via micro (at 89.2811 131.84698) (size 0.7) (drill 0.35) (layers F.Cu B.Cu) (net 5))
 (segment (start 89.2811 131.281295) (end 89.2811 129.33492) (width 0.25) (layer B.Cu) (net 5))
 (segment (start 89.2811 131.84698) (end 89.2811 131.281295) (width 0.25) (layer B.Cu) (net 5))
 (segment (start 85.60074 148.14404) (end 85.46824 148.01154) (width 0.5) (layer F.Cu) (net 5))
 (segment (start 85.60074 149.88322) (end 85.60074 148.14404) (width 0.5) (layer F.Cu) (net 5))
 (segment (start 69.05 145.85) (end 70.20316 147.00316) (width 0.25) (layer F.Cu) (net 5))
 (segment (start 67.95 145.85) (end 69.05 145.85) (width 0.25) (layer F.Cu) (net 5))
 (segment (start 70.20316 147.00316) (end 71.95068 147.00316) (width 0.25) (layer F.Cu) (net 5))
 (segment (start 72.5875 146.36634) (end 72.5875 145.5) (width 0.25) (layer F.Cu) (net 5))
 (segment (start 71.95068 147.00316) (end 72.5875 146.36634) (width 0.25) (layer F.Cu) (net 5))
 (segment (start 82.64154 150.8919) (end 82.64154 149.99528) (width 0.25) (layer F.Cu) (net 5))
 (segment (start 71.86178 150.89444) (end 85.06452 150.89444) (width 0.5) (layer F.Cu) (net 5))
 (segment (start 82.64154 149.99528) (end 82.64154 146.41134) (width 0.25) (layer B.Cu) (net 5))
 (segment (start 82.64154 140.84874) (end 82.64154 140.84874) (width 0.25) (layer B.Cu) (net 5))
 (via micro (at 82.64154 140.84874) (size 0.7) (drill 0.35) (layers F.Cu B.Cu) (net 5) (status 1000000))
 (segment (start 82.64154 140.84874) (end 83.0327 140.84874) (width 0.25) (layer F.Cu) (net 5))
 (segment (start 83.29604 141.11208) (end 83.29604 142.47378) (width 0.25) (layer F.Cu) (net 5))
 (segment (start 83.0327 140.84874) (end 83.29604 141.11208) (width 0.25) (layer F.Cu) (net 5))
 (segment (start 82.64154 146.41134) (end 82.64154 140.84874) (width 0.25) (layer B.Cu) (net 5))
 (via micro (at 82.64154 146.41134) (size 0.7) (drill 0.35) (layers F.Cu B.Cu) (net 5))
 (segment (start 89.2811 133.73928) (end 88.47592 134.54446) (width 0.25) (layer B.Cu) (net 5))
 (segment (start 89.2811 131.84698) (end 89.2811 133.73928) (width 0.25) (layer B.Cu) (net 5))
 (segment (start 87.57666 135.44372) (end 88.47592 134.54446) (width 0.25) (layer F.Cu) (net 5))
 (segment (start 87.57666 135.55112) (end 87.57666 135.44372) (width 0.25) (layer F.Cu) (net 5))
 (segment (start 82.64154 145.77552) (end 83.29604 145.12102) (width 0.25) (layer F.Cu) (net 5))
 (segment (start 82.64154 146.41134) (end 82.64154 145.77552) (width 0.25) (layer F.Cu) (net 5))
 (segment (start 79.6745 132.18906) (end 79.92678 132.44134) (width 0.25) (layer F.Cu) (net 2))
 (segment (start 79.6745 131.03906) (end 79.6745 132.18906) (width 0.25) (layer F.Cu) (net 2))
 (segment (start 79.92678 132.44134) (end 80.42666 132.44134) (width 0.25) (layer F.Cu) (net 2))
 (segment (start 80.79604 132.81072) (end 80.79604 134.14878) (width 0.25) (layer F.Cu) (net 2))
 (segment (start 80.42666 132.44134) (end 80.79604 132.81072) (width 0.25) (layer F.Cu) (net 2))
 (segment (start 79.217 131.49656) (end 79.6745 131.03906) (width 0.25) (layer F.Cu) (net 2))
 (segment (start 77.79014 131.49656) (end 79.217 131.49656) (width 0.25) (layer F.Cu) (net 2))
 (segment (start 82.1745 132.18906) (end 81.89682 132.46674) (width 0.25) (layer F.Cu) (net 1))
 (segment (start 82.1745 131.03906) (end 82.1745 132.18906) (width 0.25) (layer F.Cu) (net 1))
 (segment (start 81.89682 132.46674) (end 81.53664 132.46674) (width 0.25) (layer F.Cu) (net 1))
 (segment (start 81.29604 132.70734) (end 81.29604 134.14878) (width 0.25) (layer F.Cu) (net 1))
 (segment (start 81.53664 132.46674) (end 81.29604 132.70734) (width 0.25) (layer F.Cu) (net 1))
 (segment (start 82.632 131.49656) (end 82.1745 131.03906) (width 0.25) (layer F.Cu) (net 1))
 (segment (start 83.9471 131.49656) (end 82.632 131.49656) (width 0.25) (layer F.Cu) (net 1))
 (segment (start 85.84194 131.49656) (end 87.6047 131.49656) (width 0.25) (layer F.Cu) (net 18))
 (segment (start 93.50512 131.72316) (end 95.23078 131.72316) (width 0.25) (layer F.Cu) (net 25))
 (segment (start 93.50512 129.99464) (end 95.27078 129.99464) (width 0.25) (layer F.Cu) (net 24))
 (segment (start 67.95 140.77) (end 70.9838 140.77) (width 0.25) (layer F.Cu) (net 21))
 (segment (start 69.152081 143.31) (end 70.9838 143.31) (width 0.25) (layer F.Cu) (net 22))
 (segment (start 67.95 143.31) (end 69.152081 143.31) (width 0.25) (layer F.Cu) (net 22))
 (segment (start 91.93012 129.99464) (end 91.93012 131.72316) (width 0.25) (layer F.Cu) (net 12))
 (segment (start 78.79604 145.12102) (end 78.79604 142.47378) (width 0.25) (layer F.Cu) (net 13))
 (segment (start 77.32103 141.645588) (end 77.555348 141.41127) (width 0.25) (layer F.Cu) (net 14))
 (segment (start 74.285358 141.645588) (end 77.32103 141.645588) (width 0.25) (layer F.Cu) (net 14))
 (segment (start 73.40977 140.77) (end 74.285358 141.645588) (width 0.25) (layer F.Cu) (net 14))
 (segment (start 72.5588 140.77) (end 73.40977 140.77) (width 0.25) (layer F.Cu) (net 14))
 (segment (start 78.29604 141.73628) (end 78.29604 142.47378) (width 0.25) (layer F.Cu) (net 14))
 (segment (start 78.29604 141.670578) (end 78.29604 141.73628) (width 0.25) (layer F.Cu) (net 14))
 (segment (start 78.036732 141.41127) (end 78.29604 141.670578) (width 0.25) (layer F.Cu) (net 14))
 (segment (start 77.555348 141.41127) (end 78.036732 141.41127) (width 0.25) (layer F.Cu) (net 14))
 (segment (start 84.76936 137.56128) (end 87.57666 137.56128) (width 0.25) (layer F.Cu) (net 6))
 (segment (start 84.70854 137.56128) (end 84.76936 137.56128) (width 0.25) (layer F.Cu) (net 6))
 (segment (start 77.79604 142.47378) (end 77.79604 143.78924) (width 0.25) (layer F.Cu) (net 15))
 (segment (start 77.22104 144.36424) (end 77.22104 145.12102) (width 0.25) (layer F.Cu) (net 15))
 (segment (start 77.79604 143.78924) (end 77.22104 144.36424) (width 0.25) (layer F.Cu) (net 15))
 (segment (start 74.10714 131.49656) (end 75.994172 131.49656) (width 0.25) (layer F.Cu) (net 17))
 (segment (start 70.9838 135.69) (end 67.95 135.69) (width 0.25) (layer F.Cu) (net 19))
 (segment (start 67.95 138.23) (end 70.9838 138.23) (width 0.25) (layer F.Cu) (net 20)))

